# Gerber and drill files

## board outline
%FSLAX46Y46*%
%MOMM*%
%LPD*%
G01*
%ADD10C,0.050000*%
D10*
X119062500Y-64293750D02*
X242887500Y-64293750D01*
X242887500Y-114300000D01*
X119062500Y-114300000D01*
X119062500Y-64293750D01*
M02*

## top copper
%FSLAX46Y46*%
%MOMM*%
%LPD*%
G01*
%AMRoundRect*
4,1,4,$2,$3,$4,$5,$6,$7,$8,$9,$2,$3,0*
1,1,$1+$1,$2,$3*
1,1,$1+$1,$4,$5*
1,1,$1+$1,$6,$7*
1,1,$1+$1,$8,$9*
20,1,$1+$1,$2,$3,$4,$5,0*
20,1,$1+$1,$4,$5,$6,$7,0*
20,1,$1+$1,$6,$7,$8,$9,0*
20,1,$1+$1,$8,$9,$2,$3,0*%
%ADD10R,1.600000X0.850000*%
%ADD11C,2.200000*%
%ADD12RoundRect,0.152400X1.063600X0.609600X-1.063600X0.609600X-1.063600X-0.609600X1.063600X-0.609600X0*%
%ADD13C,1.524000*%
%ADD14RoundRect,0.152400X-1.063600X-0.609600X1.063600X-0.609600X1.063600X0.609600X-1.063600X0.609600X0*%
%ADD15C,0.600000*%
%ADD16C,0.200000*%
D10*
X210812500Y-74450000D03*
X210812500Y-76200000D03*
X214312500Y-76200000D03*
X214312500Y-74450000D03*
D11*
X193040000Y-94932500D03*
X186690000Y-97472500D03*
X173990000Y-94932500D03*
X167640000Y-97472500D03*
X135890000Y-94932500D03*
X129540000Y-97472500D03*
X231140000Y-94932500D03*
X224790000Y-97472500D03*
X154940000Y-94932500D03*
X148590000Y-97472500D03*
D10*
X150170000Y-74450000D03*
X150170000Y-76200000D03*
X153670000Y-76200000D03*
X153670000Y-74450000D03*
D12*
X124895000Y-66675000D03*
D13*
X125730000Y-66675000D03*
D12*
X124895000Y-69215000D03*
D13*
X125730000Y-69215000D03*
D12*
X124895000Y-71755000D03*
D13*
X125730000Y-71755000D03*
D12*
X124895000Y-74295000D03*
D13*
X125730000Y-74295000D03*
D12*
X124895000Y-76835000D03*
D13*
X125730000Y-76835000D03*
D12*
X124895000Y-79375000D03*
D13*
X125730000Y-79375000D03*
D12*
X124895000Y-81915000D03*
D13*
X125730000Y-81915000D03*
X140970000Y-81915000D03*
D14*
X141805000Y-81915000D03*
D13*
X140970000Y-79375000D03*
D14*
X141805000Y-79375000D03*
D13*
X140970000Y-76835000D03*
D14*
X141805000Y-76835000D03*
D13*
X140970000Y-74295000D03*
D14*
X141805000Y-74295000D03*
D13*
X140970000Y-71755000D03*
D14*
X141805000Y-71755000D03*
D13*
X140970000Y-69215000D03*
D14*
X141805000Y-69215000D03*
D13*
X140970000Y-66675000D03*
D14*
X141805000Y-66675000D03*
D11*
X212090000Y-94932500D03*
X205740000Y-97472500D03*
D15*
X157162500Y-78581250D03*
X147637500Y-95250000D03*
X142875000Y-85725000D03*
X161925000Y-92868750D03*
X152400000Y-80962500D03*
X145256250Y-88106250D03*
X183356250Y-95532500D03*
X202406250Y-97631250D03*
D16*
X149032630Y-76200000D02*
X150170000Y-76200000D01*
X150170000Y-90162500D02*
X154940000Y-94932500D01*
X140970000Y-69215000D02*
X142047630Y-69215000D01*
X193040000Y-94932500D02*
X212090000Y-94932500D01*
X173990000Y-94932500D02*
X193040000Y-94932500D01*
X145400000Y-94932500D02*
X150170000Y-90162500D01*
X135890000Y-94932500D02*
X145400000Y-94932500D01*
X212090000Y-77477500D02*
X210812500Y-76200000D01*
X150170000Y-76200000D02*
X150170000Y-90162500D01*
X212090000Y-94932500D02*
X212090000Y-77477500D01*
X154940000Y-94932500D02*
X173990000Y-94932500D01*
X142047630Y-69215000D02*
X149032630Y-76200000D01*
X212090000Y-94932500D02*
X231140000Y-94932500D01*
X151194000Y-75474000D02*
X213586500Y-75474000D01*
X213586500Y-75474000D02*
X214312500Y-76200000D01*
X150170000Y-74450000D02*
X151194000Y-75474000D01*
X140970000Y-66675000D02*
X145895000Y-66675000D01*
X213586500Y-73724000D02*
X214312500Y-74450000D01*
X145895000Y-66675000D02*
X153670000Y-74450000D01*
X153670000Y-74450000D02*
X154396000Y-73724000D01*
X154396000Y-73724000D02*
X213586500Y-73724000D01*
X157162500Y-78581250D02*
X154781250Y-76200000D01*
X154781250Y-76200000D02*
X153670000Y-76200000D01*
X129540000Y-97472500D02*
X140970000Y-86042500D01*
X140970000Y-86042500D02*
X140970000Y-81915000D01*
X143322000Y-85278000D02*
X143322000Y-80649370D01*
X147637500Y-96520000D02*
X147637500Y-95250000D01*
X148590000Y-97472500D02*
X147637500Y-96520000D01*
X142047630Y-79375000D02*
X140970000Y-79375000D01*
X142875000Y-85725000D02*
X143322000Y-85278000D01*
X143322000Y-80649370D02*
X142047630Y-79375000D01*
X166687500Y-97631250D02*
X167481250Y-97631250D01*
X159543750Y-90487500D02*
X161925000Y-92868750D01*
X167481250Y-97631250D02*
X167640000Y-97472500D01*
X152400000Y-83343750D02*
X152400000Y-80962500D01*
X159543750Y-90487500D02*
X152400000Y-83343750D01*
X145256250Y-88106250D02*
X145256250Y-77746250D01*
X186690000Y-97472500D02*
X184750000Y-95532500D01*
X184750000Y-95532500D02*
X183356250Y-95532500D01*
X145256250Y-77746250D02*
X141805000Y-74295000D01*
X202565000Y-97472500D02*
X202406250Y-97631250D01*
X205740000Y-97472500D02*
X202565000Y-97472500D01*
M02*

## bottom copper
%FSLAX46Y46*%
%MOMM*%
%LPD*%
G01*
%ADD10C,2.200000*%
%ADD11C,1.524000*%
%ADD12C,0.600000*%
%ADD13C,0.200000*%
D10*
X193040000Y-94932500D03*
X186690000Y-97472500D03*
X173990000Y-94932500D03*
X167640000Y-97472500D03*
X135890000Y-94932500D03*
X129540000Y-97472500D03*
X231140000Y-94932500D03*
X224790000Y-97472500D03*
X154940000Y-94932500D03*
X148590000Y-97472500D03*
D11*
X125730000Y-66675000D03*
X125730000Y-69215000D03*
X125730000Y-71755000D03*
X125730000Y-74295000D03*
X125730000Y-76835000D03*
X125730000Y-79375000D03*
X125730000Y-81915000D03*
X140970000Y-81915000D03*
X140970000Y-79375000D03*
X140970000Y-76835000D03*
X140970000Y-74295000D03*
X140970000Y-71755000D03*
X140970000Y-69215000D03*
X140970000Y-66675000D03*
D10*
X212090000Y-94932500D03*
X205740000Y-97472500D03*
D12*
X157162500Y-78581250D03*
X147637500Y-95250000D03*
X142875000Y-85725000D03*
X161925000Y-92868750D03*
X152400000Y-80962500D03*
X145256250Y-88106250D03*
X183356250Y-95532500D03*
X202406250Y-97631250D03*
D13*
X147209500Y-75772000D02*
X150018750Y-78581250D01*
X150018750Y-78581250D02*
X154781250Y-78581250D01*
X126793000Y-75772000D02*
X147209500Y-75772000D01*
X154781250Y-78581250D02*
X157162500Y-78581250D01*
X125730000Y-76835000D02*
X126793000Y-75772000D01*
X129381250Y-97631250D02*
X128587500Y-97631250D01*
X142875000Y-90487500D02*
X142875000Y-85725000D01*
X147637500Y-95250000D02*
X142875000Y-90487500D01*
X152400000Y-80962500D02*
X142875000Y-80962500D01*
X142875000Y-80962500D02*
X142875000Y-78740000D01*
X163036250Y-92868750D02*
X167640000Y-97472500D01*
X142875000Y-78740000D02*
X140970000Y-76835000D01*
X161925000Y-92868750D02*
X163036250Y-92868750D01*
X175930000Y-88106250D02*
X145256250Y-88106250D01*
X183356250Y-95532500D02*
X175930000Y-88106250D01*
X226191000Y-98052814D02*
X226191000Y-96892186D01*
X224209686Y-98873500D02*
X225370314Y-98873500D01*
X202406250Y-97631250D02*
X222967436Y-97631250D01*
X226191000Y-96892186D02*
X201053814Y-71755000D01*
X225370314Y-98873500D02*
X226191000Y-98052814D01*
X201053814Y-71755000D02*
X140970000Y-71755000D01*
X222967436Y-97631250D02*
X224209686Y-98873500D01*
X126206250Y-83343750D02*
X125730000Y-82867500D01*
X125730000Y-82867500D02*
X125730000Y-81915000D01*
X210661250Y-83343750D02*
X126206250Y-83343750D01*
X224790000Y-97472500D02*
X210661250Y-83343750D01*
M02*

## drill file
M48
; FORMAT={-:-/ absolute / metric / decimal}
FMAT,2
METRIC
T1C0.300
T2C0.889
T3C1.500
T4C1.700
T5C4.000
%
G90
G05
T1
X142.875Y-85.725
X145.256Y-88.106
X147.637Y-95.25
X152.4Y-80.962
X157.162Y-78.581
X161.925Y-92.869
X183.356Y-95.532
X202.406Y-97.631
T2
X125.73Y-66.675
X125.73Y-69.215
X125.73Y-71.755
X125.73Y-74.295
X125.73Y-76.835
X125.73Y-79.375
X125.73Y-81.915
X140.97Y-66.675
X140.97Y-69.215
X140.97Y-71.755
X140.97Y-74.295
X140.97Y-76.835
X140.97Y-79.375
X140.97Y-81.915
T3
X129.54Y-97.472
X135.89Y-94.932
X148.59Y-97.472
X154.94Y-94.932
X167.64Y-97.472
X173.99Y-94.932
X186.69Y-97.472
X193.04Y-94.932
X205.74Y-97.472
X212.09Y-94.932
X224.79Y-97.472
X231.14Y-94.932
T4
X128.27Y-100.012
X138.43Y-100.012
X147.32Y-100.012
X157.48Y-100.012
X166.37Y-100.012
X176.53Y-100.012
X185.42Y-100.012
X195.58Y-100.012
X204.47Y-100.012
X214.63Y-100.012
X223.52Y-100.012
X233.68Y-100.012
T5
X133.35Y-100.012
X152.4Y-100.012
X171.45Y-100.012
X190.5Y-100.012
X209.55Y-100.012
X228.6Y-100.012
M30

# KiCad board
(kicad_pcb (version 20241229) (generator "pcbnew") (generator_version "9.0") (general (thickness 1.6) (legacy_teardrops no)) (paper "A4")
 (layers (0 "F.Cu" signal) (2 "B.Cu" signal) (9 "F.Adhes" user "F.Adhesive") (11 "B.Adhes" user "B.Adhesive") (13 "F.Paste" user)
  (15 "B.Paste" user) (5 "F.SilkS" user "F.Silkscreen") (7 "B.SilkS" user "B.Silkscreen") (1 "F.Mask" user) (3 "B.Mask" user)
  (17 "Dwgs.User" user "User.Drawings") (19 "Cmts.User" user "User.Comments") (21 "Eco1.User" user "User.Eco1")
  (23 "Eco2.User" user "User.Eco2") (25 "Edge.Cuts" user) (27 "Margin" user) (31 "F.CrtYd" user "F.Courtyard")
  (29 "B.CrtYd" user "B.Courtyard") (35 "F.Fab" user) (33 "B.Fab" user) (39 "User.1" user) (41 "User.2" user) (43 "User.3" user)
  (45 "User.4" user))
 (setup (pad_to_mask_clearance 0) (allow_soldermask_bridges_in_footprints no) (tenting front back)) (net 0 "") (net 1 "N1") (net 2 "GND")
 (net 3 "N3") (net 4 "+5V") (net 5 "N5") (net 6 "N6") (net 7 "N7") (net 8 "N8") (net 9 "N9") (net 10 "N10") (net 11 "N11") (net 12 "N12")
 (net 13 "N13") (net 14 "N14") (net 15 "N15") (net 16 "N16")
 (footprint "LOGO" (layer "F.Cu") (at 169.754101 70.000013)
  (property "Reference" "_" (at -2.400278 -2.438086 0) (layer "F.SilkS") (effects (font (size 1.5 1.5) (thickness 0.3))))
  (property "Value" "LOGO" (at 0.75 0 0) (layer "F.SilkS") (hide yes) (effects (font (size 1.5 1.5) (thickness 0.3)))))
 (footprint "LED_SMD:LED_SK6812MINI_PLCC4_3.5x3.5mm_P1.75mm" (layer "F.Cu") (at 212.5625 75.325)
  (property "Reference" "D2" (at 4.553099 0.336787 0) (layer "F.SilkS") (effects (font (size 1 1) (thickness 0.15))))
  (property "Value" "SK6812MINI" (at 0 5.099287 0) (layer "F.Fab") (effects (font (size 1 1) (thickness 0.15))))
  (pad "1" smd rect (at -1.75 -0.875) (size 1.6 0.85) (layers "F.Cu" "F.Mask" "F.Paste") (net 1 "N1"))
  (pad "2" smd rect (at -1.75 0.875) (size 1.6 0.85) (layers "F.Cu" "F.Mask" "F.Paste") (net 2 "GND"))
  (pad "3" smd rect (at 1.75 0.875) (size 1.6 0.85) (layers "F.Cu" "F.Mask" "F.Paste") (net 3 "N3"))
  (pad "4" smd rect (at 1.75 -0.875) (size 1.6 0.85) (layers "F.Cu" "F.Mask" "F.Paste") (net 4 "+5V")))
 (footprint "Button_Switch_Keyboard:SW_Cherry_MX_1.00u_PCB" (layer "F.Cu") (at 193.04 94.9325)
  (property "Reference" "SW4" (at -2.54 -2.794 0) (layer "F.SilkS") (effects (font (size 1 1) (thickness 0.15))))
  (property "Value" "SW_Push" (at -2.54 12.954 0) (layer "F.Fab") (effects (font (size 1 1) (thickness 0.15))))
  (pad "" np_thru_hole circle (at -7.62 5.08) (size 1.7 1.7) (drill 1.7) (layers "*.Cu" "*.Mask"))
  (pad "" np_thru_hole circle (at -2.54 5.08) (size 4 4) (drill 4) (layers "*.Cu" "*.Mask"))
  (pad "" np_thru_hole circle (at 2.54 5.08) (size 1.7 1.7) (drill 1.7) (layers "*.Cu" "*.Mask"))
  (pad "1" thru_hole circle (at 0 0) (size 2.2 2.2) (drill 1.5) (layers "*.Cu" "*.Mask") (remove_unused_layers no) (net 2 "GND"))
  (pad "2" thru_hole circle (at -6.35 2.54) (size 2.2 2.2) (drill 1.5) (layers "*.Cu" "*.Mask") (remove_unused_layers no) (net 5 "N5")))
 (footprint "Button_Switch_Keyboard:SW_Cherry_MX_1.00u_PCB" (layer "F.Cu") (at 173.99 94.9325)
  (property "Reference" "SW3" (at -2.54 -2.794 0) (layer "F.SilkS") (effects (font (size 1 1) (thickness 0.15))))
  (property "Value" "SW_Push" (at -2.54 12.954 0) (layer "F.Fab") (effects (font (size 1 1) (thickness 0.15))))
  (pad "" np_thru_hole circle (at -7.62 5.08) (size 1.7 1.7) (drill 1.7) (layers "*.Cu" "*.Mask"))
  (pad "" np_thru_hole circle (at -2.54 5.08) (size 4 4) (drill 4) (layers "*.Cu" "*.Mask"))
  (pad "" np_thru_hole circle (at 2.54 5.08) (size 1.7 1.7) (drill 1.7) (layers "*.Cu" "*.Mask"))
  (pad "1" thru_hole circle (at 0 0) (size 2.2 2.2) (drill 1.5) (layers "*.Cu" "*.Mask") (remove_unused_layers no) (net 2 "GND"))
  (pad "2" thru_hole circle (at -6.35 2.54) (size 2.2 2.2) (drill 1.5) (layers "*.Cu" "*.Mask") (remove_unused_layers no) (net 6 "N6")))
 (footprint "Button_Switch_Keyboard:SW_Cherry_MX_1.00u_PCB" (layer "F.Cu") (at 135.89 94.9325)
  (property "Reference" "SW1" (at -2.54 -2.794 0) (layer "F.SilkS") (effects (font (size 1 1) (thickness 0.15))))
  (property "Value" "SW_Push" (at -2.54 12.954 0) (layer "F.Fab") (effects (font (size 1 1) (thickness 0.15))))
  (pad "" np_thru_hole circle (at -7.62 5.08) (size 1.7 1.7) (drill 1.7) (layers "*.Cu" "*.Mask"))
  (pad "" np_thru_hole circle (at -2.54 5.08) (size 4 4) (drill 4) (layers "*.Cu" "*.Mask"))
  (pad "" np_thru_hole circle (at 2.54 5.08) (size 1.7 1.7) (drill 1.7) (layers "*.Cu" "*.Mask"))
  (pad "1" thru_hole circle (at 0 0) (size 2.2 2.2) (drill 1.5) (layers "*.Cu" "*.Mask") (remove_unused_layers no) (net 2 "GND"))
  (pad "2" thru_hole circle (at -6.35 2.54) (size 2.2 2.2) (drill 1.5) (layers "*.Cu" "*.Mask") (remove_unused_layers no) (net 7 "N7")))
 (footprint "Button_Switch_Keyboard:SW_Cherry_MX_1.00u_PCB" (layer "F.Cu") (at 231.14 94.9325)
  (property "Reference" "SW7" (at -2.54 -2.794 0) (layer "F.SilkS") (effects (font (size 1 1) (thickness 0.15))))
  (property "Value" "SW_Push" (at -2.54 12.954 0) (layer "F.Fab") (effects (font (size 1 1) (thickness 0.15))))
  (pad "" np_thru_hole circle (at -7.62 5.08) (size 1.7 1.7) (drill 1.7) (layers "*.Cu" "*.Mask"))
  (pad "" np_thru_hole circle (at -2.54 5.08) (size 4 4) (drill 4) (layers "*.Cu" "*.Mask"))
  (pad "" np_thru_hole circle (at 2.54 5.08) (size 1.7 1.7) (drill 1.7) (layers "*.Cu" "*.Mask"))
  (pad "1" thru_hole circle (at 0 0) (size 2.2 2.2) (drill 1.5) (layers "*.Cu" "*.Mask") (remove_unused_layers no) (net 2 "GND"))
  (pad "2" thru_hole circle (at -6.35 2.54) (size 2.2 2.2) (drill 1.5) (layers "*.Cu" "*.Mask") (remove_unused_layers no) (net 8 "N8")))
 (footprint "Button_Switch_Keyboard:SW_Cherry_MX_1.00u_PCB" (layer "F.Cu") (at 154.94 94.9325)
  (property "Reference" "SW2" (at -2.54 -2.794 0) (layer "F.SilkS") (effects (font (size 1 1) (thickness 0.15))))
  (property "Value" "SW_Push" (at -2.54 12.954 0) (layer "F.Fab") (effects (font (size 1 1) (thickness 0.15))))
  (pad "" np_thru_hole circle (at -7.62 5.08) (size 1.7 1.7) (drill 1.7) (layers "*.Cu" "*.Mask"))
  (pad "" np_thru_hole circle (at -2.54 5.08) (size 4 4) (drill 4) (layers "*.Cu" "*.Mask"))
  (pad "" np_thru_hole circle (at 2.54 5.08) (size 1.7 1.7) (drill 1.7) (layers "*.Cu" "*.Mask"))
  (pad "1" thru_hole circle (at 0 0) (size 2.2 2.2) (drill 1.5) (layers "*.Cu" "*.Mask") (remove_unused_layers no) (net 2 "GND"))
  (pad "2" thru_hole circle (at -6.35 2.54) (size 2.2 2.2) (drill 1.5) (layers "*.Cu" "*.Mask") (remove_unused_layers no) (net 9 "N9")))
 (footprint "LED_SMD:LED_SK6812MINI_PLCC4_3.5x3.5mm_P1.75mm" (layer "F.Cu") (at 151.92 75.325)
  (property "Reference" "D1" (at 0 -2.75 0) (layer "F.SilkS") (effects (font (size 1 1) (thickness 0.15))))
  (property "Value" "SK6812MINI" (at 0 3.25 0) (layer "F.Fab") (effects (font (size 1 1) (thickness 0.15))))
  (pad "1" smd rect (at -1.75 -0.875) (size 1.6 0.85) (layers "F.Cu" "F.Mask" "F.Paste") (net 3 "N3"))
  (pad "2" smd rect (at -1.75 0.875) (size 1.6 0.85) (layers "F.Cu" "F.Mask" "F.Paste") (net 2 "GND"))
  (pad "3" smd rect (at 1.75 0.875) (size 1.6 0.85) (layers "F.Cu" "F.Mask" "F.Paste") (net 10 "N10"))
  (pad "4" smd rect (at 1.75 -0.875) (size 1.6 0.85) (layers "F.Cu" "F.Mask" "F.Paste") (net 4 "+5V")))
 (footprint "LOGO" (layer "F.Cu") (at 230.98125 76.2)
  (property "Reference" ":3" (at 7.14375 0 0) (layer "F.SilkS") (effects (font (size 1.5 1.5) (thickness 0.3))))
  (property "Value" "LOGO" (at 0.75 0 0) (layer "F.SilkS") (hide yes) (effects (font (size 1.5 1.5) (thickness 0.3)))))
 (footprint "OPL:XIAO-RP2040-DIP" (layer "F.Cu") (at 133.35 74.295)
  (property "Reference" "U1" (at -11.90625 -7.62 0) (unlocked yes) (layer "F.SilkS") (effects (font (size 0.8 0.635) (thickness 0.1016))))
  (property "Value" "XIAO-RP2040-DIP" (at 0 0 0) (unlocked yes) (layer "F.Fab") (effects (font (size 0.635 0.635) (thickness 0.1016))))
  (pad "1" smd roundrect (at -8.455 -7.62 180) (size 2.432 1.524) (layers "F.Cu" "F.Mask") (roundrect_rratio 0.1) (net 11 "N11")
   (thermal_bridge_angle 45))
  (pad "1" thru_hole circle (at -7.62 -7.62 180) (size 1.524 1.524) (drill 0.889) (layers "*.Cu" "*.Mask") (remove_unused_layers no)
   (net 11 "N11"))
  (pad "2" smd roundrect (at -8.455 -5.08 180) (size 2.432 1.524) (layers "F.Cu" "F.Mask") (roundrect_rratio 0.1) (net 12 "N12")
   (thermal_bridge_angle 45))
  (pad "2" thru_hole circle (at -7.62 -5.08 180) (size 1.524 1.524) (drill 0.889) (layers "*.Cu" "*.Mask") (remove_unused_layers no)
   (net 12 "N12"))
  (pad "3" smd roundrect (at -8.455 -2.54 180) (size 2.432 1.524) (layers "F.Cu" "F.Mask") (roundrect_rratio 0.1) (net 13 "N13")
   (thermal_bridge_angle 45))
  (pad "3" thru_hole circle (at -7.62 -2.54 180) (size 1.524 1.524) (drill 0.889) (layers "*.Cu" "*.Mask") (remove_unused_layers no)
   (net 13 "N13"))
  (pad "4" smd roundrect (at -8.455 0 180) (size 2.432 1.524) (layers "F.Cu" "F.Mask") (roundrect_rratio 0.1) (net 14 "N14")
   (thermal_bridge_angle 45))
  (pad "4" thru_hole circle (at -7.62 0 180) (size 1.524 1.524) (drill 0.889) (layers "*.Cu" "*.Mask") (remove_unused_layers no)
   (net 14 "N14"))
  (pad "5" smd roundrect (at -8.455 2.54 180) (size 2.432 1.524) (layers "F.Cu" "F.Mask") (roundrect_rratio 0.1) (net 10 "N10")
   (thermal_bridge_angle 45))
  (pad "5" thru_hole circle (at -7.62 2.54 180) (size 1.524 1.524) (drill 0.889) (layers "*.Cu" "*.Mask") (remove_unused_layers no)
   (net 10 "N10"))
  (pad "6" smd roundrect (at -8.455 5.08 180) (size 2.432 1.524) (layers "F.Cu" "F.Mask") (roundrect_rratio 0.1) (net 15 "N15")
   (thermal_bridge_angle 45))
  (pad "6" thru_hole circle (at -7.62 5.08 180) (size 1.524 1.524) (drill 0.889) (layers "*.Cu" "*.Mask") (remove_unused_layers no)
   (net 15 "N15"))
  (pad "7" smd roundrect (at -8.455 7.62 180) (size 2.432 1.524) (layers "F.Cu" "F.Mask") (roundrect_rratio 0.1) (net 8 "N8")
   (thermal_bridge_angle 45))
  (pad "7" thru_hole circle (at -7.62 7.62 180) (size 1.524 1.524) (drill 0.889) (layers "*.Cu" "*.Mask") (remove_unused_layers no)
   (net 8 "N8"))
  (pad "8" thru_hole circle (at 7.62 7.62) (size 1.524 1.524) (drill 0.889) (layers "*.Cu" "*.Mask") (remove_unused_layers no) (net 7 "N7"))
  (pad "8" smd roundrect (at 8.455 7.62) (size 2.432 1.524) (layers "F.Cu" "F.Mask") (roundrect_rratio 0.1) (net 7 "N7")
   (thermal_bridge_angle 45))
  (pad "9" thru_hole circle (at 7.62 5.08) (size 1.524 1.524) (drill 0.889) (layers "*.Cu" "*.Mask") (remove_unused_layers no) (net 9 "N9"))
  (pad "9" smd roundrect (at 8.455 5.08) (size 2.432 1.524) (layers "F.Cu" "F.Mask") (roundrect_rratio 0.1) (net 9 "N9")
   (thermal_bridge_angle 45))
  (pad "10" thru_hole circle (at 7.62 2.54) (size 1.524 1.524) (drill 0.889) (layers "*.Cu" "*.Mask") (remove_unused_layers no) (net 6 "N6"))
  (pad "10" smd roundrect (at 8.455 2.54) (size 2.432 1.524) (layers "F.Cu" "F.Mask") (roundrect_rratio 0.1) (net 6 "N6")
   (thermal_bridge_angle 45))
  (pad "11" thru_hole circle (at 7.62 0) (size 1.524 1.524) (drill 0.889) (layers "*.Cu" "*.Mask") (remove_unused_layers no) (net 5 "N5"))
  (pad "11" smd roundrect (at 8.455 0) (size 2.432 1.524) (layers "F.Cu" "F.Mask") (roundrect_rratio 0.1) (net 5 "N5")
   (thermal_bridge_angle 45))
  (pad "12" thru_hole circle (at 7.62 -2.54) (size 1.524 1.524) (drill 0.889) (layers "*.Cu" "*.Mask") (remove_unused_layers no)
   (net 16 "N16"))
  (pad "12" smd roundrect (at 8.455 -2.54) (size 2.432 1.524) (layers "F.Cu" "F.Mask") (roundrect_rratio 0.1) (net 16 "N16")
   (thermal_bridge_angle 45))
  (pad "13" thru_hole circle (at 7.62 -5.08) (size 1.524 1.524) (drill 0.889) (layers "*.Cu" "*.Mask") (remove_unused_layers no)
   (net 2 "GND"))
  (pad "13" smd roundrect (at 8.455 -5.08) (size 2.432 1.524) (layers "F.Cu" "F.Mask") (roundrect_rratio 0.1) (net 2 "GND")
   (thermal_bridge_angle 45))
  (pad "14" thru_hole circle (at 7.62 -7.62) (size 1.524 1.524) (drill 0.889) (layers "*.Cu" "*.Mask") (remove_unused_layers no)
   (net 4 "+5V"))
  (pad "14" smd roundrect (at 8.455 -7.62) (size 2.432 1.524) (layers "F.Cu" "F.Mask") (roundrect_rratio 0.1) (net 4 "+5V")
   (thermal_bridge_angle 45)))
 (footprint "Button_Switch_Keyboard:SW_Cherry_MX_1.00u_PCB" (layer "F.Cu") (at 212.09 94.9325)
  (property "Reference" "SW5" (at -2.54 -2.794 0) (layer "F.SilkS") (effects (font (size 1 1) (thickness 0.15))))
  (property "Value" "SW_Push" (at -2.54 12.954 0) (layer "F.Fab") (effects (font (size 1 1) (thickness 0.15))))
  (pad "" np_thru_hole circle (at -7.62 5.08) (size 1.7 1.7) (drill 1.7) (layers "*.Cu" "*.Mask"))
  (pad "" np_thru_hole circle (at -2.54 5.08) (size 4 4) (drill 4) (layers "*.Cu" "*.Mask"))
  (pad "" np_thru_hole circle (at 2.54 5.08) (size 1.7 1.7) (drill 1.7) (layers "*.Cu" "*.Mask"))
  (pad "1" thru_hole circle (at 0 0) (size 2.2 2.2) (drill 1.5) (layers "*.Cu" "*.Mask") (remove_unused_layers no) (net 2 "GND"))
  (pad "2" thru_hole circle (at -6.35 2.54) (size 2.2 2.2) (drill 1.5) (layers "*.Cu" "*.Mask") (remove_unused_layers no) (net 16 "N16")))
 (gr_rect (start 119.0625 64.29375) (end 242.8875 114.3) (stroke (width 0.05) (type default)) (fill no) (layer "Edge.Cuts"))
 (segment (start 149.03263 76.2) (end 150.17 76.2) (width 0.2) (layer "F.Cu") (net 2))
 (segment (start 150.17 90.1625) (end 154.94 94.9325) (width 0.2) (layer "F.Cu") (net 2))
 (segment (start 140.97 69.215) (end 142.04763 69.215) (width 0.2) (layer "F.Cu") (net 2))
 (segment (start 193.04 94.9325) (end 212.09 94.9325) (width 0.2) (layer "F.Cu") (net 2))
 (segment (start 173.99 94.9325) (end 193.04 94.9325) (width 0.2) (layer "F.Cu") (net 2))
 (segment (start 145.4 94.9325) (end 150.17 90.1625) (width 0.2) (layer "F.Cu") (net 2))
 (segment (start 135.89 94.9325) (end 145.4 94.9325) (width 0.2) (layer "F.Cu") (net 2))
 (segment (start 212.09 77.4775) (end 210.8125 76.2) (width 0.2) (layer "F.Cu") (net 2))
 (segment (start 150.17 76.2) (end 150.17 90.1625) (width 0.2) (layer "F.Cu") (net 2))
 (segment (start 212.09 94.9325) (end 212.09 77.4775) (width 0.2) (layer "F.Cu") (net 2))
 (segment (start 154.94 94.9325) (end 173.99 94.9325) (width 0.2) (layer "F.Cu") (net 2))
 (segment (start 142.04763 69.215) (end 149.03263 76.2) (width 0.2) (layer "F.Cu") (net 2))
 (segment (start 212.09 94.9325) (end 231.14 94.9325) (width 0.2) (layer "F.Cu") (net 2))
 (segment (start 151.194 75.474) (end 213.5865 75.474) (width 0.2) (layer "F.Cu") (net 3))
 (segment (start 213.5865 75.474) (end 214.3125 76.2) (width 0.2) (layer "F.Cu") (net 3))
 (segment (start 150.17 74.45) (end 151.194 75.474) (width 0.2) (layer "F.Cu") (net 3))
 (segment (start 140.97 66.675) (end 145.895 66.675) (width 0.2) (layer "F.Cu") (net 4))
 (segment (start 213.5865 73.724) (end 214.3125 74.45) (width 0.2) (layer "F.Cu") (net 4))
 (segment (start 145.895 66.675) (end 153.67 74.45) (width 0.2) (layer "F.Cu") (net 4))
 (segment (start 153.67 74.45) (end 154.396 73.724) (width 0.2) (layer "F.Cu") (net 4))
 (segment (start 154.396 73.724) (end 213.5865 73.724) (width 0.2) (layer "F.Cu") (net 4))
 (segment (start 157.1625 78.58125) (end 154.78125 76.2) (width 0.2) (layer "F.Cu") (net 10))
 (segment (start 154.78125 76.2) (end 153.67 76.2) (width 0.2) (layer "F.Cu") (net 10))
 (via (at 157.1625 78.58125) (size 0.6) (drill 0.3) (layers "F.Cu" "B.Cu") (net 10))
 (segment (start 147.2095 75.772) (end 150.01875 78.58125) (width 0.2) (layer "B.Cu") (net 10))
 (segment (start 150.01875 78.58125) (end 154.78125 78.58125) (width 0.2) (layer "B.Cu") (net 10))
 (segment (start 126.793 75.772) (end 147.2095 75.772) (width 0.2) (layer "B.Cu") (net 10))
 (segment (start 154.78125 78.58125) (end 157.1625 78.58125) (width 0.2) (layer "B.Cu") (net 10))
 (segment (start 125.73 76.835) (end 126.793 75.772) (width 0.2) (layer "B.Cu") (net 10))
 (segment (start 129.54 97.4725) (end 140.97 86.0425) (width 0.2) (layer "F.Cu") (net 7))
 (segment (start 140.97 86.0425) (end 140.97 81.915) (width 0.2) (layer "F.Cu") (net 7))
 (segment (start 129.38125 97.63125) (end 128.5875 97.63125) (width 0.2) (layer "B.Cu") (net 7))
 (segment (start 143.322 85.278) (end 143.322 80.64937) (width 0.2) (layer "F.Cu") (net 9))
 (segment (start 147.6375 96.52) (end 147.6375 95.25) (width 0.2) (layer "F.Cu") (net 9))
 (segment (start 148.59 97.4725) (end 147.6375 96.52) (width 0.2) (layer "F.Cu") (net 9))
 (segment (start 142.04763 79.375) (end 140.97 79.375) (width 0.2) (layer "F.Cu") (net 9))
 (segment (start 142.875 85.725) (end 143.322 85.278) (width 0.2) (layer "F.Cu") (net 9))
 (segment (start 143.322 80.64937) (end 142.04763 79.375) (width 0.2) (layer "F.Cu") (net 9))
 (via (at 147.6375 95.25) (size 0.6) (drill 0.3) (layers "F.Cu" "B.Cu") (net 9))
 (via (at 142.875 85.725) (size 0.6) (drill 0.3) (layers "F.Cu" "B.Cu") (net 9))
 (segment (start 142.875 90.4875) (end 142.875 85.725) (width 0.2) (layer "B.Cu") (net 9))
 (segment (start 147.6375 95.25) (end 142.875 90.4875) (width 0.2) (layer "B.Cu") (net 9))
 (segment (start 166.6875 97.63125) (end 167.48125 97.63125) (width 0.2) (layer "F.Cu") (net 6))
 (segment (start 159.54375 90.4875) (end 161.925 92.86875) (width 0.2) (layer "F.Cu") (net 6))
 (segment (start 167.48125 97.63125) (end 167.64 97.4725) (width 0.2) (layer "F.Cu") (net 6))
 (segment (start 152.4 83.34375) (end 152.4 80.9625) (width 0.2) (layer "F.Cu") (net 6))
 (segment (start 159.54375 90.4875) (end 152.4 83.34375) (width 0.2) (layer "F.Cu") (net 6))
 (via (at 161.925 92.86875) (size 0.6) (drill 0.3) (layers "F.Cu" "B.Cu") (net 6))
 (via (at 152.4 80.9625) (size 0.6) (drill 0.3) (layers "F.Cu" "B.Cu") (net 6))
 (segment (start 152.4 80.9625) (end 142.875 80.9625) (width 0.2) (layer "B.Cu") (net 6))
 (segment (start 142.875 80.9625) (end 142.875 78.74) (width 0.2) (layer "B.Cu") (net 6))
 (segment (start 163.03625 92.86875) (end 167.64 97.4725) (width 0.2) (layer "B.Cu") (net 6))
 (segment (start 142.875 78.74) (end 140.97 76.835) (width 0.2) (layer "B.Cu") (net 6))
 (segment (start 161.925 92.86875) (end 163.03625 92.86875) (width 0.2) (layer "B.Cu") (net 6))
 (segment (start 145.25625 88.10625) (end 145.25625 77.74625) (width 0.2) (layer "F.Cu") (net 5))
 (segment (start 186.69 97.4725) (end 184.75 95.5325) (width 0.2) (layer "F.Cu") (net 5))
 (segment (start 184.75 95.5325) (end 183.35625 95.5325) (width 0.2) (layer "F.Cu") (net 5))
 (segment (start 145.25625 77.74625) (end 141.805 74.295) (width 0.2) (layer "F.Cu") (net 5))
 (via (at 145.25625 88.10625) (size 0.6) (drill 0.3) (layers "F.Cu" "B.Cu") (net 5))
 (via (at 183.35625 95.5325) (size 0.6) (drill 0.3) (layers "F.Cu" "B.Cu") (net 5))
 (segment (start 175.93 88.10625) (end 145.25625 88.10625) (width 0.2) (layer "B.Cu") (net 5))
 (segment (start 183.35625 95.5325) (end 175.93 88.10625) (width 0.2) (layer "B.Cu") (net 5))
 (segment (start 202.565 97.4725) (end 202.40625 97.63125) (width 0.2) (layer "F.Cu") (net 16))
 (segment (start 205.74 97.4725) (end 202.565 97.4725) (width 0.2) (layer "F.Cu") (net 16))
 (via (at 202.40625 97.63125) (size 0.6) (drill 0.3) (layers "F.Cu" "B.Cu") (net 16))
 (segment (start 226.191 98.052814) (end 226.191 96.892186) (width 0.2) (layer "B.Cu") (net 16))
 (segment (start 224.209686 98.8735) (end 225.370314 98.8735) (width 0.2) (layer "B.Cu") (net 16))
 (segment (start 202.40625 97.63125) (end 222.967436 97.63125) (width 0.2) (layer "B.Cu") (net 16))
 (segment (start 226.191 96.892186) (end 201.053814 71.755) (width 0.2) (layer "B.Cu") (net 16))
 (segment (start 225.370314 98.8735) (end 226.191 98.052814) (width 0.2) (layer "B.Cu") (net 16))
 (segment (start 201.053814 71.755) (end 140.97 71.755) (width 0.2) (layer "B.Cu") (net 16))
 (segment (start 222.967436 97.63125) (end 224.209686 98.8735) (width 0.2) (layer "B.Cu") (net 16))
 (segment (start 126.20625 83.34375) (end 125.73 82.8675) (width 0.2) (layer "B.Cu") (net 8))
 (segment (start 125.73 82.8675) (end 125.73 81.915) (width 0.2) (layer "B.Cu") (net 8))
 (segment (start 210.66125 83.34375) (end 126.20625 83.34375) (width 0.2) (layer "B.Cu") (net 8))
 (segment (start 224.79 97.4725) (end 210.66125 83.34375) (width 0.2) (layer "B.Cu") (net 8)))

